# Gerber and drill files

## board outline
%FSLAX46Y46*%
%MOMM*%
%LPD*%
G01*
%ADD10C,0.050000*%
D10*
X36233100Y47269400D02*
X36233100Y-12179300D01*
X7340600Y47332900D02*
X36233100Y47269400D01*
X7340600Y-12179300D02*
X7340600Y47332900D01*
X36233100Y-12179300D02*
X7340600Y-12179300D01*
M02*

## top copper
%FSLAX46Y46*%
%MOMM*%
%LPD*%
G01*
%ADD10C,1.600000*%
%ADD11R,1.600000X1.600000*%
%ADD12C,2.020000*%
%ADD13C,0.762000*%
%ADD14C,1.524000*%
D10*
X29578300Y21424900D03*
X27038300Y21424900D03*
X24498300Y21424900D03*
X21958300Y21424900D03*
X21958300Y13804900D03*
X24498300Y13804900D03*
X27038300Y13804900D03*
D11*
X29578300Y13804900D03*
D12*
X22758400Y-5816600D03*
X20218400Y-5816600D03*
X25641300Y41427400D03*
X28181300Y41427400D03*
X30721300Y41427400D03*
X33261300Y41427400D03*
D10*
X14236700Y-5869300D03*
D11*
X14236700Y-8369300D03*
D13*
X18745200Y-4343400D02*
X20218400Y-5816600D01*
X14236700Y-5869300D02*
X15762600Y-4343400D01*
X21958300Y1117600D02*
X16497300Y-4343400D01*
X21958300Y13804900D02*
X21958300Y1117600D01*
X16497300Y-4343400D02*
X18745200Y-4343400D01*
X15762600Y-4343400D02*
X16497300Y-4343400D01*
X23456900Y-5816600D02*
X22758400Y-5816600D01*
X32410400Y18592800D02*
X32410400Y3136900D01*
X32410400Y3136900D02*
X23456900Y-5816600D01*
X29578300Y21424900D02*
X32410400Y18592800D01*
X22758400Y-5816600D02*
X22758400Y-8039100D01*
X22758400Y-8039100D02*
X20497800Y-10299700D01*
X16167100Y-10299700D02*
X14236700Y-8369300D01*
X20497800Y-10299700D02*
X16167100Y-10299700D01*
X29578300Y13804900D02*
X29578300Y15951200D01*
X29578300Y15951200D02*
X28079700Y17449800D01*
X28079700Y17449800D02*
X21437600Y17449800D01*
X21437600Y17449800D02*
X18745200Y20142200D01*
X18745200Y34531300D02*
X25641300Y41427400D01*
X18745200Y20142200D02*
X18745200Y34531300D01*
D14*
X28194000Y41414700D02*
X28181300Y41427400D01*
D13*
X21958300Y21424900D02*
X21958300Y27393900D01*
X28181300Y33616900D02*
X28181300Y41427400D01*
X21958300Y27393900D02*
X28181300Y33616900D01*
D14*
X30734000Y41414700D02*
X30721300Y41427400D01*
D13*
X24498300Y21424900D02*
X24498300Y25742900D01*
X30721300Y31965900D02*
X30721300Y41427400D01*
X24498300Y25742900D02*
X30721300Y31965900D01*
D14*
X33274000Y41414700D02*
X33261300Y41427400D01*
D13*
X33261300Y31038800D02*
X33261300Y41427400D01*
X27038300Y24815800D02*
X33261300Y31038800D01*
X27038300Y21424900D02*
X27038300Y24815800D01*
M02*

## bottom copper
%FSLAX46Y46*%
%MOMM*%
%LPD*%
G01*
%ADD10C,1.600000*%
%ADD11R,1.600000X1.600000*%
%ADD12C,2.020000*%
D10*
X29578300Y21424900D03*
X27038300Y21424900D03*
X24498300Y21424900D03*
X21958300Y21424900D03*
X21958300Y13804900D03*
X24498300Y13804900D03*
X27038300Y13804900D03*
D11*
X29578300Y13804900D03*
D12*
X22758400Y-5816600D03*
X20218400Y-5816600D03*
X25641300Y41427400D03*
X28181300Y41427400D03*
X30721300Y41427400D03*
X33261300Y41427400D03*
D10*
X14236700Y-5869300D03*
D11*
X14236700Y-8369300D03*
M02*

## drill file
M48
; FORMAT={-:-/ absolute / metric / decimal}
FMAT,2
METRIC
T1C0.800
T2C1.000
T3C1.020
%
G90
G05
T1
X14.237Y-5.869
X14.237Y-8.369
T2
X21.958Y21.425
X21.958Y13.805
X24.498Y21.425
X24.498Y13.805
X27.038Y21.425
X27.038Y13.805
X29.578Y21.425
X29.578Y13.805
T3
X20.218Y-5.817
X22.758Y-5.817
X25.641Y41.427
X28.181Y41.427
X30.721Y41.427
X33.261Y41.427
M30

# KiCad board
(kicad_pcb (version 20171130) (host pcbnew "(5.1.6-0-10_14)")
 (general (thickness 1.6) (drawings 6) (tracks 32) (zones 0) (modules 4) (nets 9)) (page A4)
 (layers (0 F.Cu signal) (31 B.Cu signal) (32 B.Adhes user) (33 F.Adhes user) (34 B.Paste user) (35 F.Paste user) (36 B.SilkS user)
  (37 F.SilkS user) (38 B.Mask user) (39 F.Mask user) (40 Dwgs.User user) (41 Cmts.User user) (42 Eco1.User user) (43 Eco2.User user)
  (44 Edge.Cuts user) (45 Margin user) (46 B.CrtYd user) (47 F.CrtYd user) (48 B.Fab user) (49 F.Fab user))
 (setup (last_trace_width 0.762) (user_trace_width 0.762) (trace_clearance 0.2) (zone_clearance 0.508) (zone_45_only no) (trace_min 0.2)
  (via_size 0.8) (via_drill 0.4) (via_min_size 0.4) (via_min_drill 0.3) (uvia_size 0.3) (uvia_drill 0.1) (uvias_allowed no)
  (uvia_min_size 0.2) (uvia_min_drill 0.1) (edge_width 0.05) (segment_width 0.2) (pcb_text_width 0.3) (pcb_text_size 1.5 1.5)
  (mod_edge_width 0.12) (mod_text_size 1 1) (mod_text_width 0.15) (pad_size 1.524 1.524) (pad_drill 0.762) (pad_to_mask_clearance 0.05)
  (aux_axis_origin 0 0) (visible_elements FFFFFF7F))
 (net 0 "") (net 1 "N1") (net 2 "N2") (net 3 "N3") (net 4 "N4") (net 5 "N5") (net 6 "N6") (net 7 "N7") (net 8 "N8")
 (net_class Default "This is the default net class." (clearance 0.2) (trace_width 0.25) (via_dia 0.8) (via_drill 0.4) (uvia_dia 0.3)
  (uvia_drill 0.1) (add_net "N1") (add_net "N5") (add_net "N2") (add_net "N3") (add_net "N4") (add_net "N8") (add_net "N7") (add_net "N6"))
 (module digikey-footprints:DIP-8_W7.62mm (layer B.Cu) (at 29.5783 -13.8049 90)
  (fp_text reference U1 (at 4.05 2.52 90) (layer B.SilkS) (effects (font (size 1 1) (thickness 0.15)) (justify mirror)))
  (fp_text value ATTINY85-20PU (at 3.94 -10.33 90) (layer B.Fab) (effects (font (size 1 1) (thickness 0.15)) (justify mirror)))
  (pad 8 thru_hole circle (at 7.62 0 90) (size 1.6 1.6) (drill 1) (layers *.Cu *.Mask) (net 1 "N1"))
  (pad 7 thru_hole circle (at 7.62 -2.54 90) (size 1.6 1.6) (drill 1) (layers *.Cu *.Mask) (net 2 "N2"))
  (pad 6 thru_hole circle (at 7.62 -5.08 90) (size 1.6 1.6) (drill 1) (layers *.Cu *.Mask) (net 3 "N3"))
  (pad 5 thru_hole circle (at 7.62 -7.62 90) (size 1.6 1.6) (drill 1) (layers *.Cu *.Mask) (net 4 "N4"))
  (pad 4 thru_hole circle (at 0 -7.62 90) (size 1.6 1.6) (drill 1) (layers *.Cu *.Mask) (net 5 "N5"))
  (pad 3 thru_hole circle (at 0 -5.08 90) (size 1.6 1.6) (drill 1) (layers *.Cu *.Mask) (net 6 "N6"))
  (pad 2 thru_hole circle (at 0 -2.54 90) (size 1.6 1.6) (drill 1) (layers *.Cu *.Mask) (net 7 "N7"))
  (pad 1 thru_hole rect (at 0 0 90) (size 1.6 1.6) (drill 1) (layers *.Cu *.Mask) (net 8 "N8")))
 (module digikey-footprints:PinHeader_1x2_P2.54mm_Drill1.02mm (layer F.Cu) (at 20.2184 5.8166)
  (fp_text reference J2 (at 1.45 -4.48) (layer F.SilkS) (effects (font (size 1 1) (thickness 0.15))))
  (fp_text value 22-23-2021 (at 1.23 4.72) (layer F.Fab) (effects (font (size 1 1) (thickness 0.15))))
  (pad 2 thru_hole circle (at 2.54 0) (size 2.02 2.02) (drill 1.02) (layers *.Cu *.Mask) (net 1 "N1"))
  (pad 1 thru_hole circle (at 0 0) (size 2.02 2.02) (drill 1.02) (layers *.Cu *.Mask) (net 5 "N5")))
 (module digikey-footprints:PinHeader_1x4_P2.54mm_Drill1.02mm (layer F.Cu) (at 33.2613 -41.4274 180)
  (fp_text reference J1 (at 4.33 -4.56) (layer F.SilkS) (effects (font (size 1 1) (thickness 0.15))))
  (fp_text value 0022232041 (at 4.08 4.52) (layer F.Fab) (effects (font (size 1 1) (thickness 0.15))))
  (pad 4 thru_hole circle (at 7.62 0 180) (size 2.02 2.02) (drill 1.02) (layers *.Cu *.Mask) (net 8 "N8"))
  (pad 3 thru_hole circle (at 5.08 0 180) (size 2.02 2.02) (drill 1.02) (layers *.Cu *.Mask) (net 4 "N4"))
  (pad 2 thru_hole circle (at 2.54 0 180) (size 2.02 2.02) (drill 1.02) (layers *.Cu *.Mask) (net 3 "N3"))
  (pad 1 thru_hole circle (at 0 0 180) (size 2.02 2.02) (drill 1.02) (layers *.Cu *.Mask) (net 2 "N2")))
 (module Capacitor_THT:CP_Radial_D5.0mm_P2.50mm (layer F.Cu) (at 14.2367 8.3693 90)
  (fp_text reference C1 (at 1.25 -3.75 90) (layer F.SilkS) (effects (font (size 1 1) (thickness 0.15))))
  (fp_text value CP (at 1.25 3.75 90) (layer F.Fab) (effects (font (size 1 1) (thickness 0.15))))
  (pad 2 thru_hole circle (at 2.5 0 90) (size 1.6 1.6) (drill 0.8) (layers *.Cu *.Mask) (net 5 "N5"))
  (pad 1 thru_hole rect (at 0 0 90) (size 1.6 1.6) (drill 0.8) (layers *.Cu *.Mask) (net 1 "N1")))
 (gr_line (start 36.2331 -47.2694) (end 36.2331 12.1793) (layer Edge.Cuts) (width 0.05))
 (gr_line (start 7.3406 -47.3329) (end 36.2331 -47.2694) (layer Edge.Cuts) (width 0.05))
 (gr_line (start 7.3406 12.1793) (end 7.3406 -47.3329) (layer Edge.Cuts) (width 0.05))
 (gr_line (start 36.2331 12.1793) (end 7.3406 12.1793) (layer Edge.Cuts) (width 0.05))
 (segment (start 18.7452 4.3434) (end 20.2184 5.8166) (width 0.762) (layer F.Cu) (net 5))
 (segment (start 14.2367 5.8693) (end 15.7626 4.3434) (width 0.762) (layer F.Cu) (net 5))
 (segment (start 21.9583 -1.1176) (end 16.4973 4.3434) (width 0.762) (layer F.Cu) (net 5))
 (segment (start 21.9583 -13.8049) (end 21.9583 -1.1176) (width 0.762) (layer F.Cu) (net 5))
 (segment (start 16.4973 4.3434) (end 18.7452 4.3434) (width 0.762) (layer F.Cu) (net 5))
 (segment (start 15.7626 4.3434) (end 16.4973 4.3434) (width 0.762) (layer F.Cu) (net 5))
 (segment (start 23.4569 5.8166) (end 22.7584 5.8166) (width 0.762) (layer F.Cu) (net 1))
 (segment (start 32.4104 -18.5928) (end 32.4104 -3.1369) (width 0.762) (layer F.Cu) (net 1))
 (segment (start 32.4104 -3.1369) (end 23.4569 5.8166) (width 0.762) (layer F.Cu) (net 1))
 (segment (start 29.5783 -21.4249) (end 32.4104 -18.5928) (width 0.762) (layer F.Cu) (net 1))
 (segment (start 22.7584 5.8166) (end 22.7584 8.0391) (width 0.762) (layer F.Cu) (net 1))
 (segment (start 22.7584 8.0391) (end 20.4978 10.2997) (width 0.762) (layer F.Cu) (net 1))
 (segment (start 16.1671 10.2997) (end 14.2367 8.3693) (width 0.762) (layer F.Cu) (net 1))
 (segment (start 20.4978 10.2997) (end 16.1671 10.2997) (width 0.762) (layer F.Cu) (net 1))
 (segment (start 29.5783 -13.8049) (end 29.5783 -15.9512) (width 0.762) (layer F.Cu) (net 8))
 (segment (start 29.5783 -15.9512) (end 28.0797 -17.4498) (width 0.762) (layer F.Cu) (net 8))
 (segment (start 28.0797 -17.4498) (end 21.4376 -17.4498) (width 0.762) (layer F.Cu) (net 8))
 (segment (start 21.4376 -17.4498) (end 18.7452 -20.1422) (width 0.762) (layer F.Cu) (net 8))
 (segment (start 18.7452 -34.5313) (end 25.6413 -41.4274) (width 0.762) (layer F.Cu) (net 8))
 (segment (start 18.7452 -20.1422) (end 18.7452 -34.5313) (width 0.762) (layer F.Cu) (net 8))
 (segment (start 28.194 -41.4147) (end 28.1813 -41.4274) (width 1.524) (layer F.Cu) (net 4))
 (segment (start 21.9583 -21.4249) (end 21.9583 -27.3939) (width 0.762) (layer F.Cu) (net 4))
 (segment (start 28.1813 -33.6169) (end 28.1813 -41.4274) (width 0.762) (layer F.Cu) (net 4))
 (segment (start 21.9583 -27.3939) (end 28.1813 -33.6169) (width 0.762) (layer F.Cu) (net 4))
 (segment (start 30.734 -41.4147) (end 30.7213 -41.4274) (width 1.524) (layer F.Cu) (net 3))
 (segment (start 24.4983 -21.4249) (end 24.4983 -25.7429) (width 0.762) (layer F.Cu) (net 3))
 (segment (start 30.7213 -31.9659) (end 30.7213 -41.4274) (width 0.762) (layer F.Cu) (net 3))
 (segment (start 24.4983 -25.7429) (end 30.7213 -31.9659) (width 0.762) (layer F.Cu) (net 3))
 (segment (start 33.274 -41.4147) (end 33.2613 -41.4274) (width 1.524) (layer F.Cu) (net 2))
 (segment (start 33.2613 -31.0388) (end 33.2613 -41.4274) (width 0.762) (layer F.Cu) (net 2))
 (segment (start 27.0383 -24.8158) (end 33.2613 -31.0388) (width 0.762) (layer F.Cu) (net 2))
 (segment (start 27.0383 -21.4249) (end 27.0383 -24.8158) (width 0.762) (layer F.Cu) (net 2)))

